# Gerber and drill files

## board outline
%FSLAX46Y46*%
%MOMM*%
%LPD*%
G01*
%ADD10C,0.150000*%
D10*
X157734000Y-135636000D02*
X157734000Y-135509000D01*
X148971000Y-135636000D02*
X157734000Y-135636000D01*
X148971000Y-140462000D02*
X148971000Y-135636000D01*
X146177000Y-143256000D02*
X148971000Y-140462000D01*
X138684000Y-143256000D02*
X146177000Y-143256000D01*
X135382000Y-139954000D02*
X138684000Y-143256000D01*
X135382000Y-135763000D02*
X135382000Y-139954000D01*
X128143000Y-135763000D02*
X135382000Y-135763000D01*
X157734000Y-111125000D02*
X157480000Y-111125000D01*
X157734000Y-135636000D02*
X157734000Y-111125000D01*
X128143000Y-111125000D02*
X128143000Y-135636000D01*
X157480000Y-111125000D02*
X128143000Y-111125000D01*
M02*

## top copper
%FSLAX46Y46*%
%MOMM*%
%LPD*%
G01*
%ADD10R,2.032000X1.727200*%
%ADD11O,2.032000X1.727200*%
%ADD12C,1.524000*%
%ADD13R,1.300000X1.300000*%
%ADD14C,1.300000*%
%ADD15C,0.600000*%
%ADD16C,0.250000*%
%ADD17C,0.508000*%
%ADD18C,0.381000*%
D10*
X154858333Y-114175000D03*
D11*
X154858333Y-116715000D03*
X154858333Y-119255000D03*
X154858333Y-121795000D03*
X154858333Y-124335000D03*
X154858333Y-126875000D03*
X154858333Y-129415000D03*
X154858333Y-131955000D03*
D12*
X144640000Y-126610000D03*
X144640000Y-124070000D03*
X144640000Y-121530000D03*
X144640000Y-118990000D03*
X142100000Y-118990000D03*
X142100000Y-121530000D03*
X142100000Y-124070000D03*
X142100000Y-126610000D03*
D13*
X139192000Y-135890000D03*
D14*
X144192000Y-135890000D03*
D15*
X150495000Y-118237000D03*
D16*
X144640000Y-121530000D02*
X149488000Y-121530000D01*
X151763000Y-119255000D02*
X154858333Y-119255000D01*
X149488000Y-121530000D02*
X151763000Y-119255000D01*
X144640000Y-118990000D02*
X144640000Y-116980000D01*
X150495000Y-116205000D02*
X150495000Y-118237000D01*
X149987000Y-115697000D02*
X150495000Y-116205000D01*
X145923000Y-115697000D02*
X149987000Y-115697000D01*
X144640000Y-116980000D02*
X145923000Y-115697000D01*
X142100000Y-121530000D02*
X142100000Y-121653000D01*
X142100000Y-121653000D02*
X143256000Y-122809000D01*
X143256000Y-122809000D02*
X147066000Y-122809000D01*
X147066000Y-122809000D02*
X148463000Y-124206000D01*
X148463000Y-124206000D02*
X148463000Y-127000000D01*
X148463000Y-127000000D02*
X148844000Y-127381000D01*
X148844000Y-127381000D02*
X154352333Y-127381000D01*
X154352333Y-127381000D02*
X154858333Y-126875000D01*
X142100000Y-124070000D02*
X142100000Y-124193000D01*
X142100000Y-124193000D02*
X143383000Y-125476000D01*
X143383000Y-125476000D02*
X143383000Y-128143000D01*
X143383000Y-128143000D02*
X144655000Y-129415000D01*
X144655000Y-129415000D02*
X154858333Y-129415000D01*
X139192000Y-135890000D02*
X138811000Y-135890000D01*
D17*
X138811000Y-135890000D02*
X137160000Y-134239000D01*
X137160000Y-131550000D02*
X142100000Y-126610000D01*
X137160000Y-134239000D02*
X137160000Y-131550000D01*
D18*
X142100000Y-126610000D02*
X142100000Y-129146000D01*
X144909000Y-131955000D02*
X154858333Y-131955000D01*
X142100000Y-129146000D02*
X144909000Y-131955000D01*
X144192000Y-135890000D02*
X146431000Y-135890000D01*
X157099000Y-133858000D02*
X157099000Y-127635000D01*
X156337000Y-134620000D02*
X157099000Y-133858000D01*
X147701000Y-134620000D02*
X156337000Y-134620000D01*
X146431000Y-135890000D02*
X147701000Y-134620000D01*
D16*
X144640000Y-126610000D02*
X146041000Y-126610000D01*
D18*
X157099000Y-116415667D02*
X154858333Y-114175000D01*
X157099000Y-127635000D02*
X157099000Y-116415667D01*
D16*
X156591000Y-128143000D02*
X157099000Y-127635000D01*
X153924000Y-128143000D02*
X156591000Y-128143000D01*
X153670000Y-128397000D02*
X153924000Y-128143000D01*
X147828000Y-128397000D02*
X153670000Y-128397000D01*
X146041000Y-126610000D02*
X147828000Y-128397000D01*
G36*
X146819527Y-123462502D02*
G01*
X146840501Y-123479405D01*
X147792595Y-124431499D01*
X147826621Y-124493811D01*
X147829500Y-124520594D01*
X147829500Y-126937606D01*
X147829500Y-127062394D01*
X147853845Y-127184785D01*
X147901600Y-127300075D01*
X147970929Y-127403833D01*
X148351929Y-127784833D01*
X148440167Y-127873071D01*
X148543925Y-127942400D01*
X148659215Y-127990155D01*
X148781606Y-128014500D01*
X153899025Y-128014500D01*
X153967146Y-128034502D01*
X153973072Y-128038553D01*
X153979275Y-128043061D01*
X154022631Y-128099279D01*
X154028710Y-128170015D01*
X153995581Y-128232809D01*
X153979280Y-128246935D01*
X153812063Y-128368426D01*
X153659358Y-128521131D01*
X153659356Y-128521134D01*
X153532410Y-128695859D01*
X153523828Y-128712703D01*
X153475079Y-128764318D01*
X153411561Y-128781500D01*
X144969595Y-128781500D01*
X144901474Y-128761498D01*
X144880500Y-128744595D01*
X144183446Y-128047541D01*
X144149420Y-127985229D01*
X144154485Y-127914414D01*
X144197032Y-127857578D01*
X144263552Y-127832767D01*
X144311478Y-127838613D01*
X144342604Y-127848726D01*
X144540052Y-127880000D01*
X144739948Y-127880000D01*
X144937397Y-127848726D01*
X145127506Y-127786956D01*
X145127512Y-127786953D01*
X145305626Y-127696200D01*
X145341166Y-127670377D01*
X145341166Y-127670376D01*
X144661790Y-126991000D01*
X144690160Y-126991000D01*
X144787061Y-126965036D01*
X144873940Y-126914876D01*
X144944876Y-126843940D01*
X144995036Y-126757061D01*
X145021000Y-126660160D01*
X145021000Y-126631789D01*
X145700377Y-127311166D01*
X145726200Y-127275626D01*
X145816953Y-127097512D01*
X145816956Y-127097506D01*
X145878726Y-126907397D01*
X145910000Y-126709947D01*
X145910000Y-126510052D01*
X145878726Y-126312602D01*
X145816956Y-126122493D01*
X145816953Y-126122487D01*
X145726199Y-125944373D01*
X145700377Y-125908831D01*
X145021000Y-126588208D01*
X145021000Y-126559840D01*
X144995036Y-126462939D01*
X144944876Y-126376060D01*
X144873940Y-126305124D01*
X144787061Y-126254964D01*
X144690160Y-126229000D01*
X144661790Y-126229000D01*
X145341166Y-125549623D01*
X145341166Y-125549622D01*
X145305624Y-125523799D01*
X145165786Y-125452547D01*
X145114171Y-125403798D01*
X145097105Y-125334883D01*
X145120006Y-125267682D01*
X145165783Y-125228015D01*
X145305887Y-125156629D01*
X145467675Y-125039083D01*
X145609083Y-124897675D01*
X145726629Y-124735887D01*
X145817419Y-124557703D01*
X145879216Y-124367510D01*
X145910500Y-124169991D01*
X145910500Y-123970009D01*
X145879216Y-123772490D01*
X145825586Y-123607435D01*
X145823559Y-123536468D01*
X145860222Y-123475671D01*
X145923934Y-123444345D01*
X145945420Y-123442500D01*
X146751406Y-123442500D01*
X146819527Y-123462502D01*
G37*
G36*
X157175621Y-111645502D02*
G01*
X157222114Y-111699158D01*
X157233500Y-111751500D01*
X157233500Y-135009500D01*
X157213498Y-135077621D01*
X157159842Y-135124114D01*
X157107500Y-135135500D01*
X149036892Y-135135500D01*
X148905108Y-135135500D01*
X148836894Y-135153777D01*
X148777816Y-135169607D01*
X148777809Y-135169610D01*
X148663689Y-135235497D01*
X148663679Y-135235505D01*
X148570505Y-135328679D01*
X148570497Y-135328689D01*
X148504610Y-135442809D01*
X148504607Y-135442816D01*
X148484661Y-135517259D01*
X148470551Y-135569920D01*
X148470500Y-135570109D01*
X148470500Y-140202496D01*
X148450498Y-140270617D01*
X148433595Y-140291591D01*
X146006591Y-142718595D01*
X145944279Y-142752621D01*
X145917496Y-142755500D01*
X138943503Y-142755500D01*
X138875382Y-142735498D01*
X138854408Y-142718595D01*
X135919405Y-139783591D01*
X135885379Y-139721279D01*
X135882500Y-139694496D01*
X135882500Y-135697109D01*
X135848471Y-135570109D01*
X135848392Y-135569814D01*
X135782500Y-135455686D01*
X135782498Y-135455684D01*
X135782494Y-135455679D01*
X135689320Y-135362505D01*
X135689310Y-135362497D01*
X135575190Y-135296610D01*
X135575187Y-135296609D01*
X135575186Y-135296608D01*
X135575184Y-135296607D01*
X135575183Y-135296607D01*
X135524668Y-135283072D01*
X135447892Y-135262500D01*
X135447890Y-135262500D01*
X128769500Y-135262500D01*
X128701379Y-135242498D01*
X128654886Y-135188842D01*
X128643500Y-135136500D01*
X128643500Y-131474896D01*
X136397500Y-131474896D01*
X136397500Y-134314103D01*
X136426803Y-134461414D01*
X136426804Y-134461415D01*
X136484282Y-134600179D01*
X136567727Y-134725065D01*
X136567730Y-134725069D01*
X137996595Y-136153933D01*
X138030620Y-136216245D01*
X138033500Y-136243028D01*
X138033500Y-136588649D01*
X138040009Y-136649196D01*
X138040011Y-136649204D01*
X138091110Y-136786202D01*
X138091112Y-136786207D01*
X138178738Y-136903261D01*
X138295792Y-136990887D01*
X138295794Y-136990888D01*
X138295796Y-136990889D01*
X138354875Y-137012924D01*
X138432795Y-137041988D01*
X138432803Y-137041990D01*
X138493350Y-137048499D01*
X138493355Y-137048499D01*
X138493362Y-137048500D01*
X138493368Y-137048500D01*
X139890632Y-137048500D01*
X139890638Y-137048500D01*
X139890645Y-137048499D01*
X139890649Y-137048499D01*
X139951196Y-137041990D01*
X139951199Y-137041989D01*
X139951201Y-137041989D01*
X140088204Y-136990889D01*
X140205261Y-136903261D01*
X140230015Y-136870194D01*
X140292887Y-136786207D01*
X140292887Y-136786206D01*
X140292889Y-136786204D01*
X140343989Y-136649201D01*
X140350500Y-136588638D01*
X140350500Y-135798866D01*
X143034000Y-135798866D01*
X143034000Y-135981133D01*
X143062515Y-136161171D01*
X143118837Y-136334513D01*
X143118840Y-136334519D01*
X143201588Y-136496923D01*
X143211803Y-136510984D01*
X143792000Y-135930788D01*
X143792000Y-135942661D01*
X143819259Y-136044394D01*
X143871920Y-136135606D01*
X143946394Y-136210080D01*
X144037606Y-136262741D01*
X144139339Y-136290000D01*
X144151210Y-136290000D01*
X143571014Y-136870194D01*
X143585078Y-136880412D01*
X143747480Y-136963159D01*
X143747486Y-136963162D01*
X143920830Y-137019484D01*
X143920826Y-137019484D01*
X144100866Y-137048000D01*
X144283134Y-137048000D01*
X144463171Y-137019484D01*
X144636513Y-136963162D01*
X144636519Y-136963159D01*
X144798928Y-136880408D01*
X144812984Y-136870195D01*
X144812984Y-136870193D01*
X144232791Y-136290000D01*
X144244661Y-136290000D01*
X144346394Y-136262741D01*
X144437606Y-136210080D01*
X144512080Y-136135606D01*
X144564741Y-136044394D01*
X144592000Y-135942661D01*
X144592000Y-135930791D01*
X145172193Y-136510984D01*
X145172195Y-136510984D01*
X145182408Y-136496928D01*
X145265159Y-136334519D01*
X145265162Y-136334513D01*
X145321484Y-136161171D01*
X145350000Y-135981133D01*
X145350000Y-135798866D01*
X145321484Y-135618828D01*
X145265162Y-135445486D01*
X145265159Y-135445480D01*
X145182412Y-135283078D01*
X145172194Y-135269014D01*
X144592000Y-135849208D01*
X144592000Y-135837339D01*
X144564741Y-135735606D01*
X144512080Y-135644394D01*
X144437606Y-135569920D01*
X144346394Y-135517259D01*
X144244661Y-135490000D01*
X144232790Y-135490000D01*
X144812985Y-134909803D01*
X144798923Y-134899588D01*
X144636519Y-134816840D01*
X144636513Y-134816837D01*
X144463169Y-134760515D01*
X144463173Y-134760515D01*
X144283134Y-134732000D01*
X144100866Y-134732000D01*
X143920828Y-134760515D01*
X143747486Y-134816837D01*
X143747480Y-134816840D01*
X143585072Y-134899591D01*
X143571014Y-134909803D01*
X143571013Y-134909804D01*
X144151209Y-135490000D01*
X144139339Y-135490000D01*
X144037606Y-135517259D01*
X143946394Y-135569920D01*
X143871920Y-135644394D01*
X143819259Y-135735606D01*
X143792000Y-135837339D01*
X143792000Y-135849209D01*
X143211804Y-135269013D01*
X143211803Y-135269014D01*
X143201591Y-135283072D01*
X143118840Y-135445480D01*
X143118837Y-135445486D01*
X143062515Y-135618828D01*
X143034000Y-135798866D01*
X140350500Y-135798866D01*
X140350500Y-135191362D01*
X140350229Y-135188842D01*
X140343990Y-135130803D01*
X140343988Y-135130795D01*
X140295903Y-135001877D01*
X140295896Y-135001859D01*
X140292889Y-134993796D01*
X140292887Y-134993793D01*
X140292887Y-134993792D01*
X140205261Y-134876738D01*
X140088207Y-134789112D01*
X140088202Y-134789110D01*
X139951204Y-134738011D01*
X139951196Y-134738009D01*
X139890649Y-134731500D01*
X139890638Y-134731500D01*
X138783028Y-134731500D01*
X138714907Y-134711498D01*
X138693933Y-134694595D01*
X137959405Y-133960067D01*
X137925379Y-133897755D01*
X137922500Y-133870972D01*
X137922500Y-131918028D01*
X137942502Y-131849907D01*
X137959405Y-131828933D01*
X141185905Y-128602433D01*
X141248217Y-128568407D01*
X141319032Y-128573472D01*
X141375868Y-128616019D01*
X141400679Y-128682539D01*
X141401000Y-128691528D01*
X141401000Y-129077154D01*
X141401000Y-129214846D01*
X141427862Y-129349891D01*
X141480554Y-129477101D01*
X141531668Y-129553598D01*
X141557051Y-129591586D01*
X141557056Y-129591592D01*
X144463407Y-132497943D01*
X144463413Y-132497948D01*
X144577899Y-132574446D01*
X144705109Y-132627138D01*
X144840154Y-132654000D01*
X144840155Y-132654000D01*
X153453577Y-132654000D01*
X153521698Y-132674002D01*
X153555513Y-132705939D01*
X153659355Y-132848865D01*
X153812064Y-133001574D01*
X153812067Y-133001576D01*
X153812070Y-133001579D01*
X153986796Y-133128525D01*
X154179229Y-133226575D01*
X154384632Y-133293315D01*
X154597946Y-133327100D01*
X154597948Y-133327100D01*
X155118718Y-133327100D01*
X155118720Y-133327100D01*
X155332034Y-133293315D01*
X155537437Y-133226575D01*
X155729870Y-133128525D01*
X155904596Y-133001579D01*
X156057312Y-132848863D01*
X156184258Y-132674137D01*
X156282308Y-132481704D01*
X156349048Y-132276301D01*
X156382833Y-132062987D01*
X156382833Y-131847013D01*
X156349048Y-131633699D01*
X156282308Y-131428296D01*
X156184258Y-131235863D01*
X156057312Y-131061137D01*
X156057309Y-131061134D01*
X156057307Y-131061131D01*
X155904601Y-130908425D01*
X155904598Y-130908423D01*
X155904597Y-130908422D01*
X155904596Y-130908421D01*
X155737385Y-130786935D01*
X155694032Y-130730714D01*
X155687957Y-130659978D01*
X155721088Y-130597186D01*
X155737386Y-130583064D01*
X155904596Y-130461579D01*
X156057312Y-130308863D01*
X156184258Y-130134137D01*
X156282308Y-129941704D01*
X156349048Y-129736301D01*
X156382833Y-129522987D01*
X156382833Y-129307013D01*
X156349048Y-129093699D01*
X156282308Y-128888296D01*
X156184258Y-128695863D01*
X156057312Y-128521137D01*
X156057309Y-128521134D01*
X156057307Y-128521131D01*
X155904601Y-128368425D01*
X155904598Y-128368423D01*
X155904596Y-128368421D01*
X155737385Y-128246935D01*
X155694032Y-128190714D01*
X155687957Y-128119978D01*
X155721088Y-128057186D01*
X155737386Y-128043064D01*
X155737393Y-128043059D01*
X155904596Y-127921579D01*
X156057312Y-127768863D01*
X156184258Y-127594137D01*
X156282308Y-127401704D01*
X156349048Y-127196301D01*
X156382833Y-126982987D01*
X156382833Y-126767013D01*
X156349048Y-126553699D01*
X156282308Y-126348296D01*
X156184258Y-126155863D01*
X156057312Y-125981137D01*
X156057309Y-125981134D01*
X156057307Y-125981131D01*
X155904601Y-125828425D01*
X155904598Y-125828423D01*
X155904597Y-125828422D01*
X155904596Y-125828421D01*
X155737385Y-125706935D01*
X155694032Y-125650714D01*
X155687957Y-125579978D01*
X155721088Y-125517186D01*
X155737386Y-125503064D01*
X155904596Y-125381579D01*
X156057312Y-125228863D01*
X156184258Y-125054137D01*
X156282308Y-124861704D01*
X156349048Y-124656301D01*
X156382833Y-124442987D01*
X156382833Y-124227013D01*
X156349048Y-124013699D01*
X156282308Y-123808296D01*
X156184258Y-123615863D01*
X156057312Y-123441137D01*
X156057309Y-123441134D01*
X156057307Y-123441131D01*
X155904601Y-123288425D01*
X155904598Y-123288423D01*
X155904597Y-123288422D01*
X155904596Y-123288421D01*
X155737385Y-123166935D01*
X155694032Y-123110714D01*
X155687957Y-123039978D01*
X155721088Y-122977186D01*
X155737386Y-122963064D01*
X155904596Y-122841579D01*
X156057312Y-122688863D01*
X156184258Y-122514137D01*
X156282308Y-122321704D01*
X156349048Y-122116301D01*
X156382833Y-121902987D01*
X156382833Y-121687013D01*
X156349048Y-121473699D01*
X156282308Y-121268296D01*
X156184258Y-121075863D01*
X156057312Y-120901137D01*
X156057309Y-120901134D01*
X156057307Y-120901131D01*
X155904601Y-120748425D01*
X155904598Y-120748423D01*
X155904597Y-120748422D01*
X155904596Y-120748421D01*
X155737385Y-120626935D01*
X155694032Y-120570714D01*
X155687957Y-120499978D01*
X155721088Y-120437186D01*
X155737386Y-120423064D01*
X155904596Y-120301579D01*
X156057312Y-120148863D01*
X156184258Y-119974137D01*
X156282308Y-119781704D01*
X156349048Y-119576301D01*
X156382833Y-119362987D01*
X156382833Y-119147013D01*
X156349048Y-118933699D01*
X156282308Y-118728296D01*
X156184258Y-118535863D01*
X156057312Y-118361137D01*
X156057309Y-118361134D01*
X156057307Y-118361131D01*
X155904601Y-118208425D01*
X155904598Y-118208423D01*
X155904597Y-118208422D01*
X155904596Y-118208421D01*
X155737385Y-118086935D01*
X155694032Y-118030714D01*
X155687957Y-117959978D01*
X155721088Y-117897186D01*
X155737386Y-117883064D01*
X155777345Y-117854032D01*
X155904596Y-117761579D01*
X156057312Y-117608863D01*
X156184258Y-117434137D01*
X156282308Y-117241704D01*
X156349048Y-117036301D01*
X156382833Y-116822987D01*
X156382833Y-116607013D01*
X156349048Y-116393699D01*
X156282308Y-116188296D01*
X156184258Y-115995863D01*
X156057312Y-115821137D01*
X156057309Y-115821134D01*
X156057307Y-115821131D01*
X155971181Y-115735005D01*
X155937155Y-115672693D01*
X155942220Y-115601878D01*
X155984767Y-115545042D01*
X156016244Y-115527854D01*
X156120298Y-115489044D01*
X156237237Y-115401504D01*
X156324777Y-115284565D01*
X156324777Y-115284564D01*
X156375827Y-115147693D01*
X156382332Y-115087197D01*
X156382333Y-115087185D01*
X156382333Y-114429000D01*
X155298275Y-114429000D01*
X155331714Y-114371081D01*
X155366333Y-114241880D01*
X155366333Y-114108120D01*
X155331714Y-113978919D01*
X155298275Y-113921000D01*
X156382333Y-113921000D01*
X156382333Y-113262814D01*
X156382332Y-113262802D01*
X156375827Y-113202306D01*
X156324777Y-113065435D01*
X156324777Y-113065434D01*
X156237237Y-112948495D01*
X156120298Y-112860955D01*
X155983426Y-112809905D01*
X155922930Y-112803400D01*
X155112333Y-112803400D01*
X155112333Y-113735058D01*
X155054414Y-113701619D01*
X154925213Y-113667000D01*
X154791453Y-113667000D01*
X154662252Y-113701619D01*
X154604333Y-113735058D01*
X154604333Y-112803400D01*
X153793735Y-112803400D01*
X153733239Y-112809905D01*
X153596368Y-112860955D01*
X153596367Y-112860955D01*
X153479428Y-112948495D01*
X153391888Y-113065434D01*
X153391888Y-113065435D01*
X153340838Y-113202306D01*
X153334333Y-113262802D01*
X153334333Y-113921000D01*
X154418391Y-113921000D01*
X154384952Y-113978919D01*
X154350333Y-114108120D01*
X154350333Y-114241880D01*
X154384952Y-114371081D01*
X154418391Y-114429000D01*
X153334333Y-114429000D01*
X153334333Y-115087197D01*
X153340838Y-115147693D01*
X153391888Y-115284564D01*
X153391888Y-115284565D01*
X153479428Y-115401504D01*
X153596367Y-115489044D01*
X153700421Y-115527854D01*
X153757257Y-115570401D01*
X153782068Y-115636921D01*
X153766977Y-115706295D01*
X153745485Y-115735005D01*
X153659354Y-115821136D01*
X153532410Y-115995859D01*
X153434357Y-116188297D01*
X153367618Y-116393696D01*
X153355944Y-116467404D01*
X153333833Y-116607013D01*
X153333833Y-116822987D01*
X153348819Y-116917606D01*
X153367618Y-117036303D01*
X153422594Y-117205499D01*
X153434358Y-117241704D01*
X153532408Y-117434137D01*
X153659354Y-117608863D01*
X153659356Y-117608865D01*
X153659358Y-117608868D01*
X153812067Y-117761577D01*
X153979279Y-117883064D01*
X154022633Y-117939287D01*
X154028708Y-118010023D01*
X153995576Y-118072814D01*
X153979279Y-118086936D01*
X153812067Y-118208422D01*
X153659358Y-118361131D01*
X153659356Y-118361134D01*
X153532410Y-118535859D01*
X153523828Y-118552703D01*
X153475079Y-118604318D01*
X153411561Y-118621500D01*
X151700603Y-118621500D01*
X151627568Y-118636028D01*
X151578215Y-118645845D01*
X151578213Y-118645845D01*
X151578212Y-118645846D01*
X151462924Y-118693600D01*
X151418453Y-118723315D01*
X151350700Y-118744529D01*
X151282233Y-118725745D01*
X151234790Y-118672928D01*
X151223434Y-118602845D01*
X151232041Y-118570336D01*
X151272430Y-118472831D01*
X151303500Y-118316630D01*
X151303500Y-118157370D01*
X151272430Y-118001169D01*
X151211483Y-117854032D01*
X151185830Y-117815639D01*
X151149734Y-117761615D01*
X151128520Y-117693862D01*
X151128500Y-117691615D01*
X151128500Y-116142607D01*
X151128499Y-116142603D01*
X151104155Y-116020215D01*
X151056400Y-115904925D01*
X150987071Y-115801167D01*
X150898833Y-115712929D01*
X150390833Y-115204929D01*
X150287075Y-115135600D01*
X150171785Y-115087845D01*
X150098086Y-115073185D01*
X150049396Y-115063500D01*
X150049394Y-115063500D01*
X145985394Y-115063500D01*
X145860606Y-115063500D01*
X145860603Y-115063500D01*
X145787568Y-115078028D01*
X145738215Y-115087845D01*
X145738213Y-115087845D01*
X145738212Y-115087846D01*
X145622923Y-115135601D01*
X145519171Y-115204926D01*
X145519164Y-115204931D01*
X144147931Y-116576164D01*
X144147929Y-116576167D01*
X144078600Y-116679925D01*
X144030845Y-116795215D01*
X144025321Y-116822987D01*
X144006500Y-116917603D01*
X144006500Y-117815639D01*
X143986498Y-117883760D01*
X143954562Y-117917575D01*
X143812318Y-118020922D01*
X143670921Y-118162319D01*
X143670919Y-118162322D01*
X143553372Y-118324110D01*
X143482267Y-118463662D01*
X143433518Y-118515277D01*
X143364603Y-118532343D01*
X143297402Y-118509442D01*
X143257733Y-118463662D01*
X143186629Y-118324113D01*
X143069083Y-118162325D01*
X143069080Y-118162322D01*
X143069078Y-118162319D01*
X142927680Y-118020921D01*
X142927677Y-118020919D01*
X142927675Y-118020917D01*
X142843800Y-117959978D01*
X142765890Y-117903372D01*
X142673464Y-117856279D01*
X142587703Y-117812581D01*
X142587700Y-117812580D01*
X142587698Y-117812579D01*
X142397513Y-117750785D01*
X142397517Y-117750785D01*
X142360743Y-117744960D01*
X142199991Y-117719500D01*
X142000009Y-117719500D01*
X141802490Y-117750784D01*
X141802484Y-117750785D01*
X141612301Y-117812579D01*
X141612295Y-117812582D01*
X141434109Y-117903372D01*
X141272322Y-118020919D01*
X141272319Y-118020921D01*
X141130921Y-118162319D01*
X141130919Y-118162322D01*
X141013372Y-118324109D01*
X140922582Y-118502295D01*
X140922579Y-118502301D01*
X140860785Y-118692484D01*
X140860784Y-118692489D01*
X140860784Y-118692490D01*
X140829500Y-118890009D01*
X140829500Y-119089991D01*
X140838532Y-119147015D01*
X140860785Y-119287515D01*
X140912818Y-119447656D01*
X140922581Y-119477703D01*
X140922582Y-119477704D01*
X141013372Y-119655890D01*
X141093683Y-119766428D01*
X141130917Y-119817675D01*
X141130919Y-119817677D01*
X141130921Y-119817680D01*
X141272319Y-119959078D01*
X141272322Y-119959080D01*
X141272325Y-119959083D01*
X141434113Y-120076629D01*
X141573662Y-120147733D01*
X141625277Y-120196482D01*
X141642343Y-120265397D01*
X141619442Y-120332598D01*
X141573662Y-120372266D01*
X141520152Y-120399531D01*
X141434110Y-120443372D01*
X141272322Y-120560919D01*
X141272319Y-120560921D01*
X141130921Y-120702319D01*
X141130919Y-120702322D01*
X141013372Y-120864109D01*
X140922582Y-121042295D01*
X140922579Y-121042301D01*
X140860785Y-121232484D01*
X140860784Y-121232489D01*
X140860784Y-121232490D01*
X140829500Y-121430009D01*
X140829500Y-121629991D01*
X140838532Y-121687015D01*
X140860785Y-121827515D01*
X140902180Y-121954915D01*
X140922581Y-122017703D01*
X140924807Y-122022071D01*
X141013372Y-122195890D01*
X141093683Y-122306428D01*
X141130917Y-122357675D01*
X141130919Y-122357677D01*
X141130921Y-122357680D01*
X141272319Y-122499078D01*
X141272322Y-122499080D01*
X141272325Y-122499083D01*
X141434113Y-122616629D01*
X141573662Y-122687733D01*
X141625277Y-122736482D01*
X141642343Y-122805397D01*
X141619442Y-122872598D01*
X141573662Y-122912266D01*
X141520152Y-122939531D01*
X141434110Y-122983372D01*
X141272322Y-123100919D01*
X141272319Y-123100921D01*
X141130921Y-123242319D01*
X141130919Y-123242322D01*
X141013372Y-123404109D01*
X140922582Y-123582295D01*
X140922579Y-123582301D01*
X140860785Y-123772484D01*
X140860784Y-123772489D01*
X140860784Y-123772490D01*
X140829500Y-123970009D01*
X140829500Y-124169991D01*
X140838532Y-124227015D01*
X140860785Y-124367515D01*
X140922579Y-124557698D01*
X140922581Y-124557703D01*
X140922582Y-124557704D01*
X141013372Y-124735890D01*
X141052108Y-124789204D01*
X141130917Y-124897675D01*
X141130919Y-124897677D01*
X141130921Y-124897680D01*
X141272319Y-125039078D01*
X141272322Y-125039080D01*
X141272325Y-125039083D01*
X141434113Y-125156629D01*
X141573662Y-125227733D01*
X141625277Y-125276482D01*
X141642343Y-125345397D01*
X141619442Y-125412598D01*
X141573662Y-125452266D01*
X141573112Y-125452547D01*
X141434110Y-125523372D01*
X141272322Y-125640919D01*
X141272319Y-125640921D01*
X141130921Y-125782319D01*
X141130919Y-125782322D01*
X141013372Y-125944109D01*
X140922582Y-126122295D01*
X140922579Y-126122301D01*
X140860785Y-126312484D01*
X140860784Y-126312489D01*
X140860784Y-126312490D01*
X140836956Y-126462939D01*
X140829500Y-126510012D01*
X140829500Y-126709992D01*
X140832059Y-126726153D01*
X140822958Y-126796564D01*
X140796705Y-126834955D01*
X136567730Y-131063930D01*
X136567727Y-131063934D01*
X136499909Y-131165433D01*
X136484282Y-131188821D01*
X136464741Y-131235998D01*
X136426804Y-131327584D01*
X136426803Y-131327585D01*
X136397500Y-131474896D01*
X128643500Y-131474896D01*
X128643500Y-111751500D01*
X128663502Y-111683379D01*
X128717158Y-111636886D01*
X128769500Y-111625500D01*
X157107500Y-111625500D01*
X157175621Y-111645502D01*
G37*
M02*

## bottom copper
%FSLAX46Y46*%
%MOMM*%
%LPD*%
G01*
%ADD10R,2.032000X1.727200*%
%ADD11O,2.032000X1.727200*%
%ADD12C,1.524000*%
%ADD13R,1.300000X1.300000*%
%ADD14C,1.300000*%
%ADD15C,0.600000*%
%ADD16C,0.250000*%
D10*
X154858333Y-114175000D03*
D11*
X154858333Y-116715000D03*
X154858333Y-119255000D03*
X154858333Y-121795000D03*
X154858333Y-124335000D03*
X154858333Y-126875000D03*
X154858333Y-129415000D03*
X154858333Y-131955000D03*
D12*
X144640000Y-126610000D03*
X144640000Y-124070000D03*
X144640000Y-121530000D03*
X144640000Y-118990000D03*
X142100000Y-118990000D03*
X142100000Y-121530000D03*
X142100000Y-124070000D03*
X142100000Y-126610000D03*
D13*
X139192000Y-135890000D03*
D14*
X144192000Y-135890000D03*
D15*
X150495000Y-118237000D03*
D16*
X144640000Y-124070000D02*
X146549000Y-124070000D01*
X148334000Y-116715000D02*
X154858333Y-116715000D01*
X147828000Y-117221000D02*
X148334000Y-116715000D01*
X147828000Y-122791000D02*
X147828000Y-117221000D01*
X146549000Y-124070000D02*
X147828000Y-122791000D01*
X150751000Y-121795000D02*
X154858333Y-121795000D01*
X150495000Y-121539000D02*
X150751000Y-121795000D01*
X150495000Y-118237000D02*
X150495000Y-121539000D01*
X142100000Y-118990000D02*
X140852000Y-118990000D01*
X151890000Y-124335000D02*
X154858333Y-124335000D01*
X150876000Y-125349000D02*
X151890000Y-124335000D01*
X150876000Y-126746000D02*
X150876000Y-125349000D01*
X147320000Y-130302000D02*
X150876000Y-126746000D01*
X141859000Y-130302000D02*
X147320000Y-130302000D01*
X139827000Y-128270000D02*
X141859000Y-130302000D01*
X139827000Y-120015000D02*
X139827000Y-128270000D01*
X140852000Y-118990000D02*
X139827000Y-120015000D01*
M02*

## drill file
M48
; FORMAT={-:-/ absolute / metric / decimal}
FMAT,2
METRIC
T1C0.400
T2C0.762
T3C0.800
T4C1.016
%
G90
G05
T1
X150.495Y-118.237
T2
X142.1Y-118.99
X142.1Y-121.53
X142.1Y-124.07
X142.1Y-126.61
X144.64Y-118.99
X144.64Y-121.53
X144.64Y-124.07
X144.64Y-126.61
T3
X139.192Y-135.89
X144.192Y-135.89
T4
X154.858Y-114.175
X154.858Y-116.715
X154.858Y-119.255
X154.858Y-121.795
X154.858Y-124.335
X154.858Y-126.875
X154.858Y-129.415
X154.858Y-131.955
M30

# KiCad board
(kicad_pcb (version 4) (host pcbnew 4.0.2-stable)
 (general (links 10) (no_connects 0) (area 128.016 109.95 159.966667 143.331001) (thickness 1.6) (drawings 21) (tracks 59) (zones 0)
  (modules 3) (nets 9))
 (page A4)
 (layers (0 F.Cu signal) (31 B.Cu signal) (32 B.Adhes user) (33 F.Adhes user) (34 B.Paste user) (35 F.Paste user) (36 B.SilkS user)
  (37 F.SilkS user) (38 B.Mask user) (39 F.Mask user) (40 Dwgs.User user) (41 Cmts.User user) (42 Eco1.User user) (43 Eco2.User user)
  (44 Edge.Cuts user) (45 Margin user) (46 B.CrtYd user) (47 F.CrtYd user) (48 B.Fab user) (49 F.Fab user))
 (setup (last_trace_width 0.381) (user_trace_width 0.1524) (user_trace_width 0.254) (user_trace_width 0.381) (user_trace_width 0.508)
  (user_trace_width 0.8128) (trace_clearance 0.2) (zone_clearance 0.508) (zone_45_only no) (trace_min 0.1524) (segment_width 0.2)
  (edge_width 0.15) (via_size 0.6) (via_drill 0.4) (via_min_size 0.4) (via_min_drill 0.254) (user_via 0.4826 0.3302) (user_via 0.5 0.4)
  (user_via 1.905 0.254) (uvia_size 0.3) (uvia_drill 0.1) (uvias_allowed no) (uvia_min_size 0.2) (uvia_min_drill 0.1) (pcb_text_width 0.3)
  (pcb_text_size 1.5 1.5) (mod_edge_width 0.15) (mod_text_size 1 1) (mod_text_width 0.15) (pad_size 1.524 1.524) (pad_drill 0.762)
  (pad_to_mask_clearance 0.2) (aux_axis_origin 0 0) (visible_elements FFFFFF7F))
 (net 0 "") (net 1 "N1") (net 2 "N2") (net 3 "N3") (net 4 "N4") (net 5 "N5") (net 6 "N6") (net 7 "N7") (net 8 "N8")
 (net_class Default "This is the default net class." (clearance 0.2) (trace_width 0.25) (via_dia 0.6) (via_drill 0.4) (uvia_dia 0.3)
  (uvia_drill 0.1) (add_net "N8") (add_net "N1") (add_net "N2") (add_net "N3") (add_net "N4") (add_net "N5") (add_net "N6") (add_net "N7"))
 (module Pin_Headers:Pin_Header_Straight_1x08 (layer F.Cu) (at 154.858333 114.175)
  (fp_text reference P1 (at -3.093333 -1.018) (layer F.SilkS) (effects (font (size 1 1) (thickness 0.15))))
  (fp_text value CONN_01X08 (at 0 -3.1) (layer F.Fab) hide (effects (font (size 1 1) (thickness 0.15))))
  (pad 1 thru_hole rect (at 0 0) (size 2.032 1.7272) (drill 1.016) (layers *.Cu *.Mask F.SilkS) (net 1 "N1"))
  (pad 2 thru_hole oval (at 0 2.54) (size 2.032 1.7272) (drill 1.016) (layers *.Cu *.Mask F.SilkS) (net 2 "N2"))
  (pad 3 thru_hole oval (at 0 5.08) (size 2.032 1.7272) (drill 1.016) (layers *.Cu *.Mask F.SilkS) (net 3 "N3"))
  (pad 4 thru_hole oval (at 0 7.62) (size 2.032 1.7272) (drill 1.016) (layers *.Cu *.Mask F.SilkS) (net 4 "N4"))
  (pad 5 thru_hole oval (at 0 10.16) (size 2.032 1.7272) (drill 1.016) (layers *.Cu *.Mask F.SilkS) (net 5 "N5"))
  (pad 6 thru_hole oval (at 0 12.7) (size 2.032 1.7272) (drill 1.016) (layers *.Cu *.Mask F.SilkS) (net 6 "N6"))
  (pad 7 thru_hole oval (at 0 15.24) (size 2.032 1.7272) (drill 1.016) (layers *.Cu *.Mask F.SilkS) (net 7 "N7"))
  (pad 8 thru_hole oval (at 0 17.78) (size 2.032 1.7272) (drill 1.016) (layers *.Cu *.Mask F.SilkS) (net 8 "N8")))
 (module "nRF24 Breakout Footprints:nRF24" (layer F.Cu) (at 135.75 122.8)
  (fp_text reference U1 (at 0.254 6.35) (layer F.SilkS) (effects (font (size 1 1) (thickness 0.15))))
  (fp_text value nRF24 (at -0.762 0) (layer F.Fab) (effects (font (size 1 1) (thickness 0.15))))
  (pad 0 thru_hole circle (at 8.89 3.81) (size 1.524 1.524) (drill 0.762) (layers *.Cu *.Mask F.SilkS) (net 1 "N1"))
  (pad 1 thru_hole circle (at 8.89 1.27) (size 1.524 1.524) (drill 0.762) (layers *.Cu *.Mask F.SilkS) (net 2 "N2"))
  (pad 2 thru_hole circle (at 8.89 -1.27) (size 1.524 1.524) (drill 0.762) (layers *.Cu *.Mask F.SilkS) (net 3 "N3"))
  (pad 3 thru_hole circle (at 8.89 -3.81) (size 1.524 1.524) (drill 0.762) (layers *.Cu *.Mask F.SilkS) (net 4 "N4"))
  (pad 4 thru_hole circle (at 6.35 -3.81) (size 1.524 1.524) (drill 0.762) (layers *.Cu *.Mask F.SilkS) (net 5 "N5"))
  (pad 5 thru_hole circle (at 6.35 -1.27) (size 1.524 1.524) (drill 0.762) (layers *.Cu *.Mask F.SilkS) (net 6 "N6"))
  (pad 6 thru_hole circle (at 6.35 1.27) (size 1.524 1.524) (drill 0.762) (layers *.Cu *.Mask F.SilkS) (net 7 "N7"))
  (pad 7 thru_hole circle (at 6.35 3.81) (size 1.524 1.524) (drill 0.762) (layers *.Cu *.Mask F.SilkS) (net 8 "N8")))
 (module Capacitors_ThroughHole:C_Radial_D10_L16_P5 (layer F.Cu) (at 139.192 135.89)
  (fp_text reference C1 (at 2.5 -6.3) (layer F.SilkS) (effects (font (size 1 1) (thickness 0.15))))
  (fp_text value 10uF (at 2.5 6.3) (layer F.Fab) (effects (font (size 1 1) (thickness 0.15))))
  (pad 1 thru_hole rect (at 0 0) (size 1.3 1.3) (drill 0.8) (layers *.Cu *.Mask F.SilkS) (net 8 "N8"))
  (pad 2 thru_hole circle (at 5 0) (size 1.3 1.3) (drill 0.8) (layers *.Cu *.Mask F.SilkS) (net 1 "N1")))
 (gr_line (start 157.734 135.636) (end 157.734 135.509) (angle 90) (layer Edge.Cuts) (width 0.15))
 (gr_line (start 148.971 135.636) (end 157.734 135.636) (angle 90) (layer Edge.Cuts) (width 0.15))
 (gr_line (start 148.971 140.462) (end 148.971 135.636) (angle 90) (layer Edge.Cuts) (width 0.15))
 (gr_line (start 146.177 143.256) (end 148.971 140.462) (angle 90) (layer Edge.Cuts) (width 0.15))
 (gr_line (start 138.684 143.256) (end 146.177 143.256) (angle 90) (layer Edge.Cuts) (width 0.15))
 (gr_line (start 135.382 139.954) (end 138.684 143.256) (angle 90) (layer Edge.Cuts) (width 0.15))
 (gr_line (start 135.382 135.763) (end 135.382 139.954) (angle 90) (layer Edge.Cuts) (width 0.15))
 (gr_line (start 128.143 135.763) (end 135.382 135.763) (angle 90) (layer Edge.Cuts) (width 0.15))
 (gr_line (start 157.734 111.125) (end 157.48 111.125) (angle 90) (layer Edge.Cuts) (width 0.15))
 (gr_line (start 157.734 135.636) (end 157.734 111.125) (angle 90) (layer Edge.Cuts) (width 0.15))
 (gr_line (start 128.143 111.125) (end 128.143 135.636) (angle 90) (layer Edge.Cuts) (width 0.15))
 (gr_line (start 157.48 111.125) (end 128.143 111.125) (angle 90) (layer Edge.Cuts) (width 0.15))
 (segment (start 144.64 124.07) (end 146.549 124.07) (width 0.25) (layer B.Cu) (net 2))
 (segment (start 148.334 116.715) (end 154.858333 116.715) (width 0.25) (layer B.Cu) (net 2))
 (segment (start 147.828 117.221) (end 148.334 116.715) (width 0.25) (layer B.Cu) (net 2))
 (segment (start 147.828 122.791) (end 147.828 117.221) (width 0.25) (layer B.Cu) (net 2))
 (segment (start 146.549 124.07) (end 147.828 122.791) (width 0.25) (layer B.Cu) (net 2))
 (segment (start 144.64 121.53) (end 149.488 121.53) (width 0.25) (layer F.Cu) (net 3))
 (segment (start 151.763 119.255) (end 154.858333 119.255) (width 0.25) (layer F.Cu) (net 3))
 (segment (start 149.488 121.53) (end 151.763 119.255) (width 0.25) (layer F.Cu) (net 3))
 (segment (start 144.64 118.99) (end 144.64 116.98) (width 0.25) (layer F.Cu) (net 4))
 (segment (start 150.751 121.795) (end 154.858333 121.795) (width 0.25) (layer B.Cu) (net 4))
 (segment (start 150.495 121.539) (end 150.751 121.795) (width 0.25) (layer B.Cu) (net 4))
 (segment (start 150.495 118.237) (end 150.495 121.539) (width 0.25) (layer B.Cu) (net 4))
 (via (at 150.495 118.237) (size 0.6) (drill 0.4) (layers F.Cu B.Cu) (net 4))
 (segment (start 150.495 116.205) (end 150.495 118.237) (width 0.25) (layer F.Cu) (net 4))
 (segment (start 149.987 115.697) (end 150.495 116.205) (width 0.25) (layer F.Cu) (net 4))
 (segment (start 145.923 115.697) (end 149.987 115.697) (width 0.25) (layer F.Cu) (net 4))
 (segment (start 144.64 116.98) (end 145.923 115.697) (width 0.25) (layer F.Cu) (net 4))
 (segment (start 142.1 118.99) (end 140.852 118.99) (width 0.25) (layer B.Cu) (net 5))
 (segment (start 151.89 124.335) (end 154.858333 124.335) (width 0.25) (layer B.Cu) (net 5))
 (segment (start 150.876 125.349) (end 151.89 124.335) (width 0.25) (layer B.Cu) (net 5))
 (segment (start 150.876 126.746) (end 150.876 125.349) (width 0.25) (layer B.Cu) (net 5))
 (segment (start 147.32 130.302) (end 150.876 126.746) (width 0.25) (layer B.Cu) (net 5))
 (segment (start 141.859 130.302) (end 147.32 130.302) (width 0.25) (layer B.Cu) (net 5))
 (segment (start 139.827 128.27) (end 141.859 130.302) (width 0.25) (layer B.Cu) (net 5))
 (segment (start 139.827 120.015) (end 139.827 128.27) (width 0.25) (layer B.Cu) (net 5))
 (segment (start 140.852 118.99) (end 139.827 120.015) (width 0.25) (layer B.Cu) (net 5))
 (segment (start 142.1 121.53) (end 142.1 121.653) (width 0.25) (layer F.Cu) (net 6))
 (segment (start 142.1 121.653) (end 143.256 122.809) (width 0.25) (layer F.Cu) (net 6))
 (segment (start 143.256 122.809) (end 147.066 122.809) (width 0.25) (layer F.Cu) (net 6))
 (segment (start 147.066 122.809) (end 148.463 124.206) (width 0.25) (layer F.Cu) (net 6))
 (segment (start 148.463 124.206) (end 148.463 127) (width 0.25) (layer F.Cu) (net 6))
 (segment (start 148.463 127) (end 148.844 127.381) (width 0.25) (layer F.Cu) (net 6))
 (segment (start 148.844 127.381) (end 154.352333 127.381) (width 0.25) (layer F.Cu) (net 6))
 (segment (start 154.352333 127.381) (end 154.858333 126.875) (width 0.25) (layer F.Cu) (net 6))
 (segment (start 142.1 124.07) (end 142.1 124.193) (width 0.25) (layer F.Cu) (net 7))
 (segment (start 142.1 124.193) (end 143.383 125.476) (width 0.25) (layer F.Cu) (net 7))
 (segment (start 143.383 125.476) (end 143.383 128.143) (width 0.25) (layer F.Cu) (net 7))
 (segment (start 143.383 128.143) (end 144.655 129.415) (width 0.25) (layer F.Cu) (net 7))
 (segment (start 144.655 129.415) (end 154.858333 129.415) (width 0.25) (layer F.Cu) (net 7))
 (segment (start 139.192 135.89) (end 138.811 135.89) (width 0.25) (layer F.Cu) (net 8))
 (segment (start 138.811 135.89) (end 137.16 134.239) (width 0.508) (layer F.Cu) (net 8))
 (segment (start 137.16 131.55) (end 142.1 126.61) (width 0.508) (layer F.Cu) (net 8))
 (segment (start 137.16 134.239) (end 137.16 131.55) (width 0.508) (layer F.Cu) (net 8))
 (segment (start 142.1 126.61) (end 142.1 129.146) (width 0.381) (layer F.Cu) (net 8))
 (segment (start 144.909 131.955) (end 154.858333 131.955) (width 0.381) (layer F.Cu) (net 8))
 (segment (start 142.1 129.146) (end 144.909 131.955) (width 0.381) (layer F.Cu) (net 8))
 (segment (start 144.192 135.89) (end 146.431 135.89) (width 0.381) (layer F.Cu) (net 1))
 (segment (start 157.099 133.858) (end 157.099 127.635) (width 0.381) (layer F.Cu) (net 1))
 (segment (start 156.337 134.62) (end 157.099 133.858) (width 0.381) (layer F.Cu) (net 1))
 (segment (start 147.701 134.62) (end 156.337 134.62) (width 0.381) (layer F.Cu) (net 1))
 (segment (start 146.431 135.89) (end 147.701 134.62) (width 0.381) (layer F.Cu) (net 1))
 (segment (start 144.64 126.61) (end 146.041 126.61) (width 0.25) (layer F.Cu) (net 1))
 (segment (start 157.099 116.415667) (end 154.858333 114.175) (width 0.381) (layer F.Cu) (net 1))
 (segment (start 157.099 127.635) (end 157.099 116.415667) (width 0.381) (layer F.Cu) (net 1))
 (segment (start 156.591 128.143) (end 157.099 127.635) (width 0.25) (layer F.Cu) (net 1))
 (segment (start 153.924 128.143) (end 156.591 128.143) (width 0.25) (layer F.Cu) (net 1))
 (segment (start 153.67 128.397) (end 153.924 128.143) (width 0.25) (layer F.Cu) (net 1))
 (segment (start 147.828 128.397) (end 153.67 128.397) (width 0.25) (layer F.Cu) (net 1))
 (segment (start 146.041 126.61) (end 147.828 128.397) (width 0.25) (layer F.Cu) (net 1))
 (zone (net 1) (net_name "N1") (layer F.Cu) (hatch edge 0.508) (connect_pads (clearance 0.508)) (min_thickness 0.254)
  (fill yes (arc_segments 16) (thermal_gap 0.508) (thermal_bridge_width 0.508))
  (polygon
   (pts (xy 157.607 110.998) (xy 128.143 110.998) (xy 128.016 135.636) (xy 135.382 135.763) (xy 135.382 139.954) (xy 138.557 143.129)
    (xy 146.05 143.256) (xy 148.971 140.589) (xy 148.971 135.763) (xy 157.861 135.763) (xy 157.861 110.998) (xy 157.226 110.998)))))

